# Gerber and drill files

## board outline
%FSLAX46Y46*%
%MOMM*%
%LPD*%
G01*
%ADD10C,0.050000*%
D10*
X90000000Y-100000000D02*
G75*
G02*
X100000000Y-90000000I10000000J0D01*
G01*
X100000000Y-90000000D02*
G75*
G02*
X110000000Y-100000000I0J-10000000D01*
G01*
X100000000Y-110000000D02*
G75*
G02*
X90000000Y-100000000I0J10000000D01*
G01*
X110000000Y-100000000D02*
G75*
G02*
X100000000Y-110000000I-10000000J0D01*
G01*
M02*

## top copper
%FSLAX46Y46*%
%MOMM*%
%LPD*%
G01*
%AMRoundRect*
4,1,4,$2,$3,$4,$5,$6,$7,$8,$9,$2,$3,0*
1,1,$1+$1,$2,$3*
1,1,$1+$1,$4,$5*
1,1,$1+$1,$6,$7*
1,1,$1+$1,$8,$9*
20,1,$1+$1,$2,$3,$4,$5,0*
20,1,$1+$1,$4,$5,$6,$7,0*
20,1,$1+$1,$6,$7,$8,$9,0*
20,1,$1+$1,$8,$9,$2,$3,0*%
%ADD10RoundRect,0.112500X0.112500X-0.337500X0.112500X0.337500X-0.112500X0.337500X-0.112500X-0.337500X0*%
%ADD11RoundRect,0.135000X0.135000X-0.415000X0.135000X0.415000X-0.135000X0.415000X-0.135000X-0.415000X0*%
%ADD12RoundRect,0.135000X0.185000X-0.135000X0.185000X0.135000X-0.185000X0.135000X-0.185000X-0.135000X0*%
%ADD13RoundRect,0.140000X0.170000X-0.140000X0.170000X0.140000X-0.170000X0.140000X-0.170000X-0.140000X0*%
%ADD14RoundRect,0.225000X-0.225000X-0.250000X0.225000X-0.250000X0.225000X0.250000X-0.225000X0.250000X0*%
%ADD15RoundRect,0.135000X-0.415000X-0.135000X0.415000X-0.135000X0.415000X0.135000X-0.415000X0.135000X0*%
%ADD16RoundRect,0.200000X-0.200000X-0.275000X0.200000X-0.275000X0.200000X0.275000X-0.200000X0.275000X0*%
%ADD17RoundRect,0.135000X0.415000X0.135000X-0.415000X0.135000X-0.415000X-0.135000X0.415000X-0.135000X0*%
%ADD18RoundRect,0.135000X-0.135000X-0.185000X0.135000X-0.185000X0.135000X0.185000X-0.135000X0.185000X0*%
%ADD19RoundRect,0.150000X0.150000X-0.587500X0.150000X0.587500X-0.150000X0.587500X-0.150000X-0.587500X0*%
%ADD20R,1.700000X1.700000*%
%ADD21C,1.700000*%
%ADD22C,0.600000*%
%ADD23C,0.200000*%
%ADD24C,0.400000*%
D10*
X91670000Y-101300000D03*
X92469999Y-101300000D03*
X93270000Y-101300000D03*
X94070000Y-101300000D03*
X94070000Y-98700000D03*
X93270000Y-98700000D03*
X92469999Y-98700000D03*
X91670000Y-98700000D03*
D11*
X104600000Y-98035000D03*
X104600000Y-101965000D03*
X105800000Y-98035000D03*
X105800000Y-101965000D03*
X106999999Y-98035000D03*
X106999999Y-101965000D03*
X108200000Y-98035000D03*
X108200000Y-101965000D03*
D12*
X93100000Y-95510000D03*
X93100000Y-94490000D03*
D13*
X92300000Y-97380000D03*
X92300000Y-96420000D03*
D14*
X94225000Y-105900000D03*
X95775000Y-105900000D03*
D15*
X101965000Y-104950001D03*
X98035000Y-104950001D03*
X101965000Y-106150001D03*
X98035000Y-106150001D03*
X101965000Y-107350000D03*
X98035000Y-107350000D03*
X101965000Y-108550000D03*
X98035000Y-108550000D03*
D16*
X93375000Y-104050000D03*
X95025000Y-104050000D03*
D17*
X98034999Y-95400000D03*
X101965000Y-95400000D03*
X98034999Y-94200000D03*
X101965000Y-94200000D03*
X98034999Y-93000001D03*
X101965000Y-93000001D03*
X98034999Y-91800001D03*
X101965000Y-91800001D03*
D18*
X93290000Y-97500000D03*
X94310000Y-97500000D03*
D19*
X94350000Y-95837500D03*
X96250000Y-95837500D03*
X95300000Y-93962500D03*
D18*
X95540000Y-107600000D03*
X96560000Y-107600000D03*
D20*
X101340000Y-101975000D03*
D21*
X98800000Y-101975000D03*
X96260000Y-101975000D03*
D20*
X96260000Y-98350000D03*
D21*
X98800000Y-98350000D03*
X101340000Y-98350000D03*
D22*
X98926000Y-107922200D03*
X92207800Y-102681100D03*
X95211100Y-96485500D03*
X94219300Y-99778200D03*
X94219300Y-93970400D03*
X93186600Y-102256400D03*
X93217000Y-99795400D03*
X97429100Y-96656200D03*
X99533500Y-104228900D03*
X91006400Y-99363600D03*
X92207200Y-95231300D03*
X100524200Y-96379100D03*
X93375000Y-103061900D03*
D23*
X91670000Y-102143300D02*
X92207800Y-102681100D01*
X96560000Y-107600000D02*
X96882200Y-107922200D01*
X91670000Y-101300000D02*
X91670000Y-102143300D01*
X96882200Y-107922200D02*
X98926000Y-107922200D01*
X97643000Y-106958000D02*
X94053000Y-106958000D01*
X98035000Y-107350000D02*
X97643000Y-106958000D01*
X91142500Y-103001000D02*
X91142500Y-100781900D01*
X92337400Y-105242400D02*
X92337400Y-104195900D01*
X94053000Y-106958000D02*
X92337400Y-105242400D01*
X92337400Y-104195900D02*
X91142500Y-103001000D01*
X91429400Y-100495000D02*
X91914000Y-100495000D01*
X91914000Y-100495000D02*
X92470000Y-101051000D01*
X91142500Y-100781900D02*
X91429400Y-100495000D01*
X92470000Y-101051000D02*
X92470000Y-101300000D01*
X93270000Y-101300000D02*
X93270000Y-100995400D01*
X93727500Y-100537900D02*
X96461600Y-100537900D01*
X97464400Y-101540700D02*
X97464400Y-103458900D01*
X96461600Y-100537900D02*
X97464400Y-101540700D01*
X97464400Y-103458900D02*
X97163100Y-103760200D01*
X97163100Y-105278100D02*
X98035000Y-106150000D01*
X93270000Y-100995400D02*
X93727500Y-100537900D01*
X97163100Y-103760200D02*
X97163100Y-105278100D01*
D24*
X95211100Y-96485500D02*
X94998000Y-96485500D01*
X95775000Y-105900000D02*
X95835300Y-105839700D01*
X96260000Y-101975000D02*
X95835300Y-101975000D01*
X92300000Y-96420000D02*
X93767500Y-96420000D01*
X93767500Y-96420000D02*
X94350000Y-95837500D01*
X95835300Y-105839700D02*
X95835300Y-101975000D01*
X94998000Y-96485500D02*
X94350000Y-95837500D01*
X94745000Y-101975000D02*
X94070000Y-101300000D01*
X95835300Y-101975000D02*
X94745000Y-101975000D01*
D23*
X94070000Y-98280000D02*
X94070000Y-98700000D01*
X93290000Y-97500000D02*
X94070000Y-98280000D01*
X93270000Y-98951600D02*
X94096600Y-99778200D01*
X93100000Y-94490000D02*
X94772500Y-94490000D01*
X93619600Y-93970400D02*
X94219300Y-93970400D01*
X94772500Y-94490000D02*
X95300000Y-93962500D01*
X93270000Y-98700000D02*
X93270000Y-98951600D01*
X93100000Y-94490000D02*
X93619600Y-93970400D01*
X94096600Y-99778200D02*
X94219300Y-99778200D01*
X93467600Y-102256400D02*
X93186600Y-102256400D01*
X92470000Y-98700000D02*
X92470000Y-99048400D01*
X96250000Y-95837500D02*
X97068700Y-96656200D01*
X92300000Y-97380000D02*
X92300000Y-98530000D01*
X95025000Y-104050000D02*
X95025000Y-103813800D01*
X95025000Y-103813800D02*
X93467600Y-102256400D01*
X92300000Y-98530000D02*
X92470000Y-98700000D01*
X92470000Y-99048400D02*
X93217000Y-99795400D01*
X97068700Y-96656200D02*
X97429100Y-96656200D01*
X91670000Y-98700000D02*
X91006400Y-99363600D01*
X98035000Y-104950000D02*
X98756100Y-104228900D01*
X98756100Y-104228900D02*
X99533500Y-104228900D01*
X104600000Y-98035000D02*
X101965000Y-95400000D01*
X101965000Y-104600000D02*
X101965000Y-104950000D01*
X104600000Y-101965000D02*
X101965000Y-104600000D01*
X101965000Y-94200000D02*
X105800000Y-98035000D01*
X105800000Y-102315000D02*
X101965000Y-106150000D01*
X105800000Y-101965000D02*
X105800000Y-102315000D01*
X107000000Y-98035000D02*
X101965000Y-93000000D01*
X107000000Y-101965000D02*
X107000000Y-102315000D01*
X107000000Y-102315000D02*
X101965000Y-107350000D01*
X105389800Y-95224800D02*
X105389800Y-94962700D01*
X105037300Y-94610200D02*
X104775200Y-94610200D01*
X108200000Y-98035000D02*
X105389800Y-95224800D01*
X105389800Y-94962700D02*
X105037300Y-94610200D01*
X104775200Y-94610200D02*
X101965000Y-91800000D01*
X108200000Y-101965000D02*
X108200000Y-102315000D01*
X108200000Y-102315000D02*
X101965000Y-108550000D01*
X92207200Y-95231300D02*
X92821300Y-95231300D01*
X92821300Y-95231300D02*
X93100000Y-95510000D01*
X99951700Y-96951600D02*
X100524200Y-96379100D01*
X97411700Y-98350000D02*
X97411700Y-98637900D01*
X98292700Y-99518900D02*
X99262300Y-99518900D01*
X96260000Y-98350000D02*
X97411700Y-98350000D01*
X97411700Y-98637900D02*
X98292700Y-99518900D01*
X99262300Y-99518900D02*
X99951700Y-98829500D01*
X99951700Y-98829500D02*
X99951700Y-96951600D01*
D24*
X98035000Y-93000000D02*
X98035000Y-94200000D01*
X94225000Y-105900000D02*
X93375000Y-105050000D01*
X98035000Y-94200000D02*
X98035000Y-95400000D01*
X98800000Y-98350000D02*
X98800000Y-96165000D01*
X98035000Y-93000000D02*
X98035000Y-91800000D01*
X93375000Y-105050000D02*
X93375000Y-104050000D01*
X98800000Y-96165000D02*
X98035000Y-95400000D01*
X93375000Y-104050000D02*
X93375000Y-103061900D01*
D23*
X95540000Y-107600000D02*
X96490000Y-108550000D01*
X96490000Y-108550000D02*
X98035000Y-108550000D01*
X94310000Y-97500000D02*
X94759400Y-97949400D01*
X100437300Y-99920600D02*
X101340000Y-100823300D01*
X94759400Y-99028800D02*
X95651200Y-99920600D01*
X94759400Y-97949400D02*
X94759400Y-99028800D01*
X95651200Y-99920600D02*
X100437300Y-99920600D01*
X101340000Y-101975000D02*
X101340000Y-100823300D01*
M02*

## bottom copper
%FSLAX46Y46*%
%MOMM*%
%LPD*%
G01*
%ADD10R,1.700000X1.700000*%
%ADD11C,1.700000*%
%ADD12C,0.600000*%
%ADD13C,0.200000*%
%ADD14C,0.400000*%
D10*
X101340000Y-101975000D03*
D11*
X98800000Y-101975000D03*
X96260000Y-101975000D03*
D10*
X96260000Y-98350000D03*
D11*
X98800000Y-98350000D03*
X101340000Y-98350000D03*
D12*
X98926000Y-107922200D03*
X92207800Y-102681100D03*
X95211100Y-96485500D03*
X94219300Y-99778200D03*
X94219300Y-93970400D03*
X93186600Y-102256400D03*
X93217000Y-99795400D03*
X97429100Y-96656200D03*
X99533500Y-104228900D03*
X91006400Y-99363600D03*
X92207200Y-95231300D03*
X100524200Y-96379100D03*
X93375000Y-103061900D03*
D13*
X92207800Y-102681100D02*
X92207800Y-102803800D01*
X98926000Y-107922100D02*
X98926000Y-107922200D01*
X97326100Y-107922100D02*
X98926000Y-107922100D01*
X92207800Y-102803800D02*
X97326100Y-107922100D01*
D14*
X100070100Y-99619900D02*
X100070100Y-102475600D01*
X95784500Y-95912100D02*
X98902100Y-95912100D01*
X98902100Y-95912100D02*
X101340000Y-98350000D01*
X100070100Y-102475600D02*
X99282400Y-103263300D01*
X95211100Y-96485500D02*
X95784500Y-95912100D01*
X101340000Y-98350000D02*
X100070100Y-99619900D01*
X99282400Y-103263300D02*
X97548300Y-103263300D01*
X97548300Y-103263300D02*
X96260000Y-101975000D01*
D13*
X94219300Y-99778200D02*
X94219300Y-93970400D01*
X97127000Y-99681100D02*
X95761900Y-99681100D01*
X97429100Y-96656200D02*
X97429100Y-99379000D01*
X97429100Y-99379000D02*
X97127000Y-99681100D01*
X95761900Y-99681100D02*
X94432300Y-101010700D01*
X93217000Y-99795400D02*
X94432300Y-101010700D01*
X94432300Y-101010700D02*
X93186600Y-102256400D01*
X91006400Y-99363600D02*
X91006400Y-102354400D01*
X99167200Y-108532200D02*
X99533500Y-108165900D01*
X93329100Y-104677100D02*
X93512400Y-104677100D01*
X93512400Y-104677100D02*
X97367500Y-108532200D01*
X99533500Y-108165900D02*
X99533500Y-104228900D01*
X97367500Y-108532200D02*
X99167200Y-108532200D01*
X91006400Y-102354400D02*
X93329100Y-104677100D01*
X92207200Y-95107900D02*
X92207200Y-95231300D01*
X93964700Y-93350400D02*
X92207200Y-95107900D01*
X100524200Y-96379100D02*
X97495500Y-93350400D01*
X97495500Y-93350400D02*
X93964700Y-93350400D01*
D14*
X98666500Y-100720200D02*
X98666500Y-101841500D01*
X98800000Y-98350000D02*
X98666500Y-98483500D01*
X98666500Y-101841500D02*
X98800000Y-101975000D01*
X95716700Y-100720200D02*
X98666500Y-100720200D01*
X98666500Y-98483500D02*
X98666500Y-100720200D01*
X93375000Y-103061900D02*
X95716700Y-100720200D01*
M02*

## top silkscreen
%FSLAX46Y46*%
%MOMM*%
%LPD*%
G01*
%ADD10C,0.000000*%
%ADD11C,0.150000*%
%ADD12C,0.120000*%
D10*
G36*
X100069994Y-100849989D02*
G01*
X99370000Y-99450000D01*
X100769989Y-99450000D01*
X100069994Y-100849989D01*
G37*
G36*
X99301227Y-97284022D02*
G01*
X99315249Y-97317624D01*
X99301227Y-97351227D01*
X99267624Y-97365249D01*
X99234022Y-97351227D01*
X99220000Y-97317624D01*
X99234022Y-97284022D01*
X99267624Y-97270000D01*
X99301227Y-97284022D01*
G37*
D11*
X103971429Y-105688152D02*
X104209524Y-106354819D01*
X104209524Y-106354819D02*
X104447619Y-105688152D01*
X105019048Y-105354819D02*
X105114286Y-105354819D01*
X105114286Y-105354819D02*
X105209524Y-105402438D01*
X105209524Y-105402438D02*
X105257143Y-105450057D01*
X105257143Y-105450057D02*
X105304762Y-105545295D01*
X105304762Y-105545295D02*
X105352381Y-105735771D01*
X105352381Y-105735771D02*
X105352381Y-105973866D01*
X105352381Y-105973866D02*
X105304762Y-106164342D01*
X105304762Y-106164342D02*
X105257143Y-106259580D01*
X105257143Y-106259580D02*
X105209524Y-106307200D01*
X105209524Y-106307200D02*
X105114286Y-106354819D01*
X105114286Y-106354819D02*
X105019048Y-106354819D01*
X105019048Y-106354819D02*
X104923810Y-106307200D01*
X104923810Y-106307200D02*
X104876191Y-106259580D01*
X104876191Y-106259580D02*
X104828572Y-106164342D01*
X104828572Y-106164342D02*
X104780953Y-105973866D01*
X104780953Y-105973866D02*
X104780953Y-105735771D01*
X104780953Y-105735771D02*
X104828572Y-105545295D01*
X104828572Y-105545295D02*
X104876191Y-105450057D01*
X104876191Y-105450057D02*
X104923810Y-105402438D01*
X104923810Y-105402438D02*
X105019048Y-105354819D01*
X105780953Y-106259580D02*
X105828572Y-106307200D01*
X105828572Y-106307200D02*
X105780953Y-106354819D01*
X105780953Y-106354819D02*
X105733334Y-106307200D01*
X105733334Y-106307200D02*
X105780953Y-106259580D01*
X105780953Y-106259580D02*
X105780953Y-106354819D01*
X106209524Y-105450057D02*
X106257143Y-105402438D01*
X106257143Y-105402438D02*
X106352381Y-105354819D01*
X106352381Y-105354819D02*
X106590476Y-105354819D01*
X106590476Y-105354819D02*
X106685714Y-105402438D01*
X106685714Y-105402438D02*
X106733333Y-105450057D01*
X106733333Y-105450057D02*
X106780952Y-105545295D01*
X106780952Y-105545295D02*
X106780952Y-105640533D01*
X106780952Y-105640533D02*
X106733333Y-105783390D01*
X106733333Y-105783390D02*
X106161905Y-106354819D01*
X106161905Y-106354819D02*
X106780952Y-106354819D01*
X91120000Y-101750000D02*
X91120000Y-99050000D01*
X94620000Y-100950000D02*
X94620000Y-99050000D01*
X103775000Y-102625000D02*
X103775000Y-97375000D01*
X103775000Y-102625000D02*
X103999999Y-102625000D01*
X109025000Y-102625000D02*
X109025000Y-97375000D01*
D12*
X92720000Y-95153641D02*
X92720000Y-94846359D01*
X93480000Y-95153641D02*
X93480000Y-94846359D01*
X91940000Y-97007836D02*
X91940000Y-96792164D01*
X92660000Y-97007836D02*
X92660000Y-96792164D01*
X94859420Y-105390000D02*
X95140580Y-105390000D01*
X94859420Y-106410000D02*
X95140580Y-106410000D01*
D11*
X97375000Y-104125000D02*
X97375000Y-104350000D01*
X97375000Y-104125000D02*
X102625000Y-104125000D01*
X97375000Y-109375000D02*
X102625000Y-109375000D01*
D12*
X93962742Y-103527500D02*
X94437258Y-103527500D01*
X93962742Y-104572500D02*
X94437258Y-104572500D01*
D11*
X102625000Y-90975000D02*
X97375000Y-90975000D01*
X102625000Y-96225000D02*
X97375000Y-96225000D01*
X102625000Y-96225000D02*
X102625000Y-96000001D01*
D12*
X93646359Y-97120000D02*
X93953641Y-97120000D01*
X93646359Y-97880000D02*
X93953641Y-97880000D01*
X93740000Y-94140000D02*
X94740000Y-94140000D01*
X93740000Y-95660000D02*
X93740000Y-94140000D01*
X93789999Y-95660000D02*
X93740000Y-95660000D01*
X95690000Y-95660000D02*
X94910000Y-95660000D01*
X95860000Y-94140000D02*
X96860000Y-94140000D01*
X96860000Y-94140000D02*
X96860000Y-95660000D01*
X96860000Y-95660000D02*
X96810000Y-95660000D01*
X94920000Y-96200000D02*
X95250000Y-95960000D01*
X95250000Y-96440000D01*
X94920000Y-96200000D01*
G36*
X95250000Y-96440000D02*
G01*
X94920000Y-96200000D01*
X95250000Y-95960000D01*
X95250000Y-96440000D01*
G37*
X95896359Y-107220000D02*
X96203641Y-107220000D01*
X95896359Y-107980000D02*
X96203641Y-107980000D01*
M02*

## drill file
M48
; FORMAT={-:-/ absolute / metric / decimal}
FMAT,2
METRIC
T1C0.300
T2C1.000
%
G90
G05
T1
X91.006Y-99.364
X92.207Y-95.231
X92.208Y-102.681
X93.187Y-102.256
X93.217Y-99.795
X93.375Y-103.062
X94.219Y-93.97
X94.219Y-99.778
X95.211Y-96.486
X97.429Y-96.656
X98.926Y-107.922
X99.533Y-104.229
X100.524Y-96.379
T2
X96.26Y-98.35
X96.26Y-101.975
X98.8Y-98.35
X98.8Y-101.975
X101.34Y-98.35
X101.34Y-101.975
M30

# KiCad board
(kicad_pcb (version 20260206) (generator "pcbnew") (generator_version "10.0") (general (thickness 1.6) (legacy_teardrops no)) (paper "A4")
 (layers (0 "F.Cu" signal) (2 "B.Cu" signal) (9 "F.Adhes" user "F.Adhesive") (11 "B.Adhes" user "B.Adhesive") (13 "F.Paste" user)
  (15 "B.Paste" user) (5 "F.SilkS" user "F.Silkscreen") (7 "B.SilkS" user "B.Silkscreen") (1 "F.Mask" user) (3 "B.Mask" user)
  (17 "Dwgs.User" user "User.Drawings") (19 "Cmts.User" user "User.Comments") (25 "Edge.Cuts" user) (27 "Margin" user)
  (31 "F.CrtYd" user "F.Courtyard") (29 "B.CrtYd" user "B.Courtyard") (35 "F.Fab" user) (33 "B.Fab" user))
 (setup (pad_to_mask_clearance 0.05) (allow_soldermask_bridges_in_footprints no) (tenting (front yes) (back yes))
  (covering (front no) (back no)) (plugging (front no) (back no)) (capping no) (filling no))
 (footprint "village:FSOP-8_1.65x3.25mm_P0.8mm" (layer "F.Cu") (at 92.87 100 90)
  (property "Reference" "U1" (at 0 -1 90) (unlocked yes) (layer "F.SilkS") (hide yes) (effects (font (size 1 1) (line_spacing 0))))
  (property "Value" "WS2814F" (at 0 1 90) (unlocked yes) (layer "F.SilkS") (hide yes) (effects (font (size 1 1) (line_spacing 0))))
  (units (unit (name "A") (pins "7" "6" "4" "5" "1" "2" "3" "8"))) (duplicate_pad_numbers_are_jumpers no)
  (fp_line (start -1.75 -1.75) (end 0.95 -1.75) (stroke (width 0.15) (type solid)) (layer "F.SilkS"))
  (fp_line (start -0.95 1.75) (end 0.95 1.75) (stroke (width 0.15) (type solid)) (layer "F.SilkS"))
  (pad "1" smd roundrect (at -1.3 -1.2 90) (size 0.9 0.45) (layers "F.Cu" "F.Mask" "F.Paste") (roundrect_rratio 0.25) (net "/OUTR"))
  (pad "2" smd roundrect (at -1.3 -0.400001 90) (size 0.9 0.45) (layers "F.Cu" "F.Mask" "F.Paste") (roundrect_rratio 0.25) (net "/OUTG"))
  (pad "3" smd roundrect (at -1.3 0.4 90) (size 0.9 0.45) (layers "F.Cu" "F.Mask" "F.Paste") (roundrect_rratio 0.25) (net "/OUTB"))
  (pad "4" smd roundrect (at -1.3 1.2 90) (size 0.9 0.45) (layers "F.Cu" "F.Mask" "F.Paste") (roundrect_rratio 0.25) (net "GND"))
  (pad "5" smd roundrect (at 1.3 1.2 90) (size 0.9 0.45) (layers "F.Cu" "F.Mask" "F.Paste") (roundrect_rratio 0.25) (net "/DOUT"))
  (pad "6" smd roundrect (at 1.3 0.4 90) (size 0.9 0.45) (layers "F.Cu" "F.Mask" "F.Paste") (roundrect_rratio 0.25) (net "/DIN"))
  (pad "7" smd roundrect (at 1.3 -0.400001 90) (size 0.9 0.45) (layers "F.Cu" "F.Mask" "F.Paste") (roundrect_rratio 0.25) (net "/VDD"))
  (pad "8" smd roundrect (at 1.3 -1.2 90) (size 0.9 0.45) (layers "F.Cu" "F.Mask" "F.Paste") (roundrect_rratio 0.25) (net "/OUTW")))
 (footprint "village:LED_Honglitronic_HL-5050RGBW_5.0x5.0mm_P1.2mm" (layer "F.Cu") (at 106.4 100 90)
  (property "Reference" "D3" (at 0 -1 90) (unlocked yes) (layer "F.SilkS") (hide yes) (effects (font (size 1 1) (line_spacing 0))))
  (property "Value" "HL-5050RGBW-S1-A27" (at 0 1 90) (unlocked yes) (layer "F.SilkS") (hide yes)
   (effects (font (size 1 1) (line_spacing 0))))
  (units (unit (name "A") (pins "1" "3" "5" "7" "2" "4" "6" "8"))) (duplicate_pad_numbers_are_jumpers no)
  (fp_line (start -2.625 -2.625) (end 2.625 -2.625) (stroke (width 0.15) (type default)) (layer "F.SilkS"))
  (fp_line (start -2.625 -2.625) (end -2.625 -2.400001) (stroke (width 0.15) (type default)) (layer "F.SilkS"))
  (fp_line (start -2.625 2.625) (end 2.625 2.625) (stroke (width 0.15) (type default)) (layer "F.SilkS"))
  (pad "1" smd roundrect (at 1.965 -1.8 90) (size 1.1 0.54) (layers "F.Cu" "F.Mask" "F.Paste") (roundrect_rratio 0.25) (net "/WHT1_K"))
  (pad "2" smd roundrect (at -1.965 -1.8 90) (size 1.1 0.54) (layers "F.Cu" "F.Mask" "F.Paste") (roundrect_rratio 0.25) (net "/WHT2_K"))
  (pad "3" smd roundrect (at 1.965 -0.6 90) (size 1.1 0.54) (layers "F.Cu" "F.Mask" "F.Paste") (roundrect_rratio 0.25) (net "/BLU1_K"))
  (pad "4" smd roundrect (at -1.965 -0.6 90) (size 1.1 0.54) (layers "F.Cu" "F.Mask" "F.Paste") (roundrect_rratio 0.25) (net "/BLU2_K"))
  (pad "5" smd roundrect (at 1.965 0.599999 90) (size 1.1 0.54) (layers "F.Cu" "F.Mask" "F.Paste") (roundrect_rratio 0.25) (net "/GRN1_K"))
  (pad "6" smd roundrect (at -1.965 0.599999 90) (size 1.1 0.54) (layers "F.Cu" "F.Mask" "F.Paste") (roundrect_rratio 0.25) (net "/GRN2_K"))
  (pad "7" smd roundrect (at 1.965 1.8 90) (size 1.1 0.54) (layers "F.Cu" "F.Mask" "F.Paste") (roundrect_rratio 0.25) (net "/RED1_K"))
  (pad "8" smd roundrect (at -1.965 1.8 90) (size 1.1 0.54) (layers "F.Cu" "F.Mask" "F.Paste") (roundrect_rratio 0.25) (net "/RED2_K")))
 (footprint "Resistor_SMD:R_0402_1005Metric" (layer "F.Cu") (at 93.1 95 90)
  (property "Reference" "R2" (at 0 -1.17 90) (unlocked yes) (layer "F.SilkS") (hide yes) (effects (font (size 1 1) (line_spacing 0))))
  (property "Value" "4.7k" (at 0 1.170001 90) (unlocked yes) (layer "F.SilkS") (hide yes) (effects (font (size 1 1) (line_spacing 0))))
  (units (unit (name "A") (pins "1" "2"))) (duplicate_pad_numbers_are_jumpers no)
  (fp_line (start -0.153641 -0.38) (end 0.153641 -0.38) (stroke (width 0.12) (type solid)) (layer "F.SilkS"))
  (fp_line (start -0.153641 0.38) (end 0.153641 0.38) (stroke (width 0.12) (type solid)) (layer "F.SilkS"))
  (pad "1" smd roundrect (at -0.51 0 90) (size 0.54 0.64) (layers "F.Cu" "F.Mask" "F.Paste") (roundrect_rratio 0.25) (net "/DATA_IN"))
  (pad "2" smd roundrect (at 0.51 0 90) (size 0.54 0.64) (layers "F.Cu" "F.Mask" "F.Paste") (roundrect_rratio 0.25) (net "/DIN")))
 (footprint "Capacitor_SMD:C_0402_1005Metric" (layer "F.Cu") (at 92.3 96.9 90)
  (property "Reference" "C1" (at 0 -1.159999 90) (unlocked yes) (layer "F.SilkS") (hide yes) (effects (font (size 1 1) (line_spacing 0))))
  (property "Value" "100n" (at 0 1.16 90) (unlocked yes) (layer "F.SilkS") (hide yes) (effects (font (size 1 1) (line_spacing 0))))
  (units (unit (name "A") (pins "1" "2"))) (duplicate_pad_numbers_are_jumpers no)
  (fp_line (start -0.107836 -0.36) (end 0.107836 -0.36) (stroke (width 0.12) (type solid)) (layer "F.SilkS"))
  (fp_line (start -0.107836 0.36) (end 0.107836 0.36) (stroke (width 0.12) (type solid)) (layer "F.SilkS"))
  (pad "1" smd roundrect (at -0.48 0 90) (size 0.56 0.62) (layers "F.Cu" "F.Mask" "F.Paste") (roundrect_rratio 0.25) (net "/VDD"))
  (pad "2" smd roundrect (at 0.48 0 90) (size 0.56 0.62) (layers "F.Cu" "F.Mask" "F.Paste") (roundrect_rratio 0.25) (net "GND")))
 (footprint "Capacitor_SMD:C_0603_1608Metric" (layer "F.Cu") (at 95 105.9)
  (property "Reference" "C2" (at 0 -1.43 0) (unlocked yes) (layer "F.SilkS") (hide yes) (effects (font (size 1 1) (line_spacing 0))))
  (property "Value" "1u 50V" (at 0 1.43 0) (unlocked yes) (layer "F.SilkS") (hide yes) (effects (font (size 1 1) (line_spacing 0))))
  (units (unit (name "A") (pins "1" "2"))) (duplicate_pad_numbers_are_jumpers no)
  (fp_line (start -0.14058 -0.51) (end 0.14058 -0.51) (stroke (width 0.12) (type solid)) (layer "F.SilkS"))
  (fp_line (start -0.14058 0.51) (end 0.14058 0.51) (stroke (width 0.12) (type solid)) (layer "F.SilkS"))
  (pad "1" smd roundrect (at -0.775 0) (size 0.9 0.95) (layers "F.Cu" "F.Mask" "F.Paste") (roundrect_rratio 0.25) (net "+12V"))
  (pad "2" smd roundrect (at 0.775 0) (size 0.9 0.95) (layers "F.Cu" "F.Mask" "F.Paste") (roundrect_rratio 0.25) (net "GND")))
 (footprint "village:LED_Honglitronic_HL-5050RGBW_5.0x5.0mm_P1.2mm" (layer "F.Cu") (at 100 106.75)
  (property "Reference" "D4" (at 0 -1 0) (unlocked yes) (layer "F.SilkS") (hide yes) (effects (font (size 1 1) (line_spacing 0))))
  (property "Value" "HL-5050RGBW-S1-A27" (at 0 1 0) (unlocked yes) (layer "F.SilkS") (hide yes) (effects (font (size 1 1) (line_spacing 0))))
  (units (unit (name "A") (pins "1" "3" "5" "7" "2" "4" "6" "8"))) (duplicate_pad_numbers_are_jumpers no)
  (fp_line (start -2.625 -2.625) (end -2.625 -2.4) (stroke (width 0.15) (type default)) (layer "F.SilkS"))
  (fp_line (start -2.625 -2.625) (end 2.625 -2.625) (stroke (width 0.15) (type default)) (layer "F.SilkS"))
  (fp_line (start -2.625 2.625) (end 2.625 2.625) (stroke (width 0.15) (type default)) (layer "F.SilkS"))
  (pad "1" smd roundrect (at 1.965 -1.799999) (size 1.1 0.54) (layers "F.Cu" "F.Mask" "F.Paste") (roundrect_rratio 0.25) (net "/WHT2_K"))
  (pad "2" smd roundrect (at -1.965 -1.799999) (size 1.1 0.54) (layers "F.Cu" "F.Mask" "F.Paste") (roundrect_rratio 0.25) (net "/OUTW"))
  (pad "3" smd roundrect (at 1.965 -0.599999) (size 1.1 0.54) (layers "F.Cu" "F.Mask" "F.Paste") (roundrect_rratio 0.25) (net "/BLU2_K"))
  (pad "4" smd roundrect (at -1.965 -0.599999) (size 1.1 0.54) (layers "F.Cu" "F.Mask" "F.Paste") (roundrect_rratio 0.25) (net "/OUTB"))
  (pad "5" smd roundrect (at 1.965 0.6) (size 1.1 0.54) (layers "F.Cu" "F.Mask" "F.Paste") (roundrect_rratio 0.25) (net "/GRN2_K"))
  (pad "6" smd roundrect (at -1.965 0.6) (size 1.1 0.54) (layers "F.Cu" "F.Mask" "F.Paste") (roundrect_rratio 0.25) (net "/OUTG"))
  (pad "7" smd roundrect (at 1.965 1.8) (size 1.1 0.54) (layers "F.Cu" "F.Mask" "F.Paste") (roundrect_rratio 0.25) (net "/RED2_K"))
  (pad "8" smd roundrect (at -1.965 1.8) (size 1.1 0.54) (layers "F.Cu" "F.Mask" "F.Paste") (roundrect_rratio 0.25) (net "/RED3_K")))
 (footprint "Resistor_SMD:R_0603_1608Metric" (layer "F.Cu") (at 94.2 104.05)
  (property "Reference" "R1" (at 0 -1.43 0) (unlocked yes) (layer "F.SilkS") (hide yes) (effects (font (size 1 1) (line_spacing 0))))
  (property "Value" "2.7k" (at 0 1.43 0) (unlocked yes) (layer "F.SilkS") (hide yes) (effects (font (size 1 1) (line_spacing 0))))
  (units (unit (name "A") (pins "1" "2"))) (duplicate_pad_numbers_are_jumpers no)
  (fp_line (start -0.237258 -0.5225) (end 0.237258 -0.5225) (stroke (width 0.12) (type solid)) (layer "F.SilkS"))
  (fp_line (start -0.237258 0.5225) (end 0.237258 0.5225) (stroke (width 0.12) (type solid)) (layer "F.SilkS"))
  (pad "1" smd roundrect (at -0.825 0) (size 0.8 0.95) (layers "F.Cu" "F.Mask" "F.Paste") (roundrect_rratio 0.25) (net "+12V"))
  (pad "2" smd roundrect (at 0.825 0) (size 0.8 0.95) (layers "F.Cu" "F.Mask" "F.Paste") (roundrect_rratio 0.25) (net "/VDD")))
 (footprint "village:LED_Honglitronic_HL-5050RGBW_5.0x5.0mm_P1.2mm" (layer "F.Cu") (at 100 93.6 180)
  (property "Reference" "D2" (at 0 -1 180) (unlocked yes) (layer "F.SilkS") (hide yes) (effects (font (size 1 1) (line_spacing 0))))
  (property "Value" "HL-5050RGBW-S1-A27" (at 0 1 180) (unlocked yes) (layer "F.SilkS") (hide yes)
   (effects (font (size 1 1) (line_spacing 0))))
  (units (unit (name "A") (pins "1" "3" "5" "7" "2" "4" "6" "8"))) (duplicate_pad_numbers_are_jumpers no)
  (fp_line (start -2.625 2.625) (end 2.625 2.625) (stroke (width 0.15) (type default)) (layer "F.SilkS"))
  (fp_line (start -2.625 -2.625) (end 2.625 -2.625) (stroke (width 0.15) (type default)) (layer "F.SilkS"))
  (fp_line (start -2.625 -2.625) (end -2.625 -2.400001) (stroke (width 0.15) (type default)) (layer "F.SilkS"))
  (pad "1" smd roundrect (at 1.965001 -1.8 180) (size 1.1 0.54) (layers "F.Cu" "F.Mask" "F.Paste") (roundrect_rratio 0.25) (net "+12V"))
  (pad "2" smd roundrect (at -1.965 -1.8 180) (size 1.1 0.54) (layers "F.Cu" "F.Mask" "F.Paste") (roundrect_rratio 0.25) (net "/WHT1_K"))
  (pad "3" smd roundrect (at 1.965001 -0.6 180) (size 1.1 0.54) (layers "F.Cu" "F.Mask" "F.Paste") (roundrect_rratio 0.25) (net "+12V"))
  (pad "4" smd roundrect (at -1.965 -0.6 180) (size 1.1 0.54) (layers "F.Cu" "F.Mask" "F.Paste") (roundrect_rratio 0.25) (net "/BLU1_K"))
  (pad "5" smd roundrect (at 1.965001 0.599999 180) (size 1.1 0.54) (layers "F.Cu" "F.Mask" "F.Paste") (roundrect_rratio 0.25) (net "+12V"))
  (pad "6" smd roundrect (at -1.965 0.599999 180) (size 1.1 0.54) (layers "F.Cu" "F.Mask" "F.Paste") (roundrect_rratio 0.25) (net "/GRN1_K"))
  (pad "7" smd roundrect (at 1.965001 1.799999 180) (size 1.1 0.54) (layers "F.Cu" "F.Mask" "F.Paste") (roundrect_rratio 0.25) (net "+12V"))
  (pad "8" smd roundrect (at -1.965 1.799999 180) (size 1.1 0.54) (layers "F.Cu" "F.Mask" "F.Paste") (roundrect_rratio 0.25) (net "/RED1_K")))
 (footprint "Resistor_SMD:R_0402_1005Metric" (layer "F.Cu") (at 93.8 97.5)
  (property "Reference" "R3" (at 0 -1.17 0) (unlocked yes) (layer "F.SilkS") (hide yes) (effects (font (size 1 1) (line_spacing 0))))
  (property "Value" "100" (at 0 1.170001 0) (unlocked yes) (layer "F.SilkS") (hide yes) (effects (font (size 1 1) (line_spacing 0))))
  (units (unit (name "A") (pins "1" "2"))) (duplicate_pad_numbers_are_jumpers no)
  (fp_line (start -0.153641 -0.38) (end 0.153641 -0.38) (stroke (width 0.12) (type solid)) (layer "F.SilkS"))
  (fp_line (start -0.153641 0.38) (end 0.153641 0.38) (stroke (width 0.12) (type solid)) (layer "F.SilkS"))
  (pad "1" smd roundrect (at -0.51 0) (size 0.54 0.64) (layers "F.Cu" "F.Mask" "F.Paste") (roundrect_rratio 0.25) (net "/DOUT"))
  (pad "2" smd roundrect (at 0.51 0) (size 0.54 0.64) (layers "F.Cu" "F.Mask" "F.Paste") (roundrect_rratio 0.25) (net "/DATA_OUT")))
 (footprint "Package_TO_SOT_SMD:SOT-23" (layer "F.Cu") (at 95.3 94.9 90)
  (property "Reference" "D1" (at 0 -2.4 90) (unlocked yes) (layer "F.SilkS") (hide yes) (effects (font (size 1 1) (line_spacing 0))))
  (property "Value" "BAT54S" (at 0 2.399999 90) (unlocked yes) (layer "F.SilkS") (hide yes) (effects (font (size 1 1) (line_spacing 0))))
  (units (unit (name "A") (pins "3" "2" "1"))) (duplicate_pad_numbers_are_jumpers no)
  (fp_line (start 0.76 -1.56) (end 0.76 -0.56) (stroke (width 0.12) (type solid)) (layer "F.SilkS"))
  (fp_line (start -0.76 -1.56) (end 0.76 -1.56) (stroke (width 0.12) (type solid)) (layer "F.SilkS"))
  (fp_line (start -0.76 -1.510001) (end -0.76 -1.56) (stroke (width 0.12) (type solid)) (layer "F.SilkS"))
  (fp_line (start -0.76 0.39) (end -0.76 -0.39) (stroke (width 0.12) (type solid)) (layer "F.SilkS"))
  (fp_line (start 0.76 0.56) (end 0.76 1.56) (stroke (width 0.12) (type solid)) (layer "F.SilkS"))
  (fp_line (start 0.76 1.56) (end -0.76 1.56) (stroke (width 0.12) (type solid)) (layer "F.SilkS"))
  (fp_line (start -0.76 1.56) (end -0.76 1.51) (stroke (width 0.12) (type solid)) (layer "F.SilkS"))
  (fp_poly (pts (xy -1.3 -0.38) (xy -1.06 -0.05) (xy -1.54 -0.05)) (stroke (width 0.12) (type solid)) (fill yes) (layer "F.SilkS"))
  (pad "1" smd roundrect (at -0.9375 -0.95 90) (size 1.475 0.6) (layers "F.Cu" "F.Mask" "F.Paste") (roundrect_rratio 0.25) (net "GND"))
  (pad "2" smd roundrect (at -0.9375 0.95 90) (size 1.475 0.6) (layers "F.Cu" "F.Mask" "F.Paste") (roundrect_rratio 0.25) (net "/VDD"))
  (pad "3" smd roundrect (at 0.9375 0 90) (size 1.475 0.6) (layers "F.Cu" "F.Mask" "F.Paste") (roundrect_rratio 0.25) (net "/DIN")))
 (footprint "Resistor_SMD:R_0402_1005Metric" (layer "F.Cu") (at 96.05 107.6)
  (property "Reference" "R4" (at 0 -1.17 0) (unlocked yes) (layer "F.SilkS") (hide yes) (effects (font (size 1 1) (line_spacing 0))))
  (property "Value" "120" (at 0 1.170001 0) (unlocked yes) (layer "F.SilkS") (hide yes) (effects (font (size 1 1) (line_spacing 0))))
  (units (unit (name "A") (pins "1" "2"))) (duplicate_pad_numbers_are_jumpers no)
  (fp_line (start -0.153641 -0.38) (end 0.153641 -0.38) (stroke (width 0.12) (type solid)) (layer "F.SilkS"))
  (fp_line (start -0.153641 0.38) (end 0.153641 0.38) (stroke (width 0.12) (type solid)) (layer "F.SilkS"))
  (pad "1" smd roundrect (at -0.51 0) (size 0.54 0.64) (layers "F.Cu" "F.Mask" "F.Paste") (roundrect_rratio 0.25) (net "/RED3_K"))
  (pad "2" smd roundrect (at 0.51 0) (size 0.54 0.64) (layers "F.Cu" "F.Mask" "F.Paste") (roundrect_rratio 0.25) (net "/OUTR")))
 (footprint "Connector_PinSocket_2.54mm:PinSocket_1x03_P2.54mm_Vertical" (layer "B.Cu") (at 101.34 101.975 90)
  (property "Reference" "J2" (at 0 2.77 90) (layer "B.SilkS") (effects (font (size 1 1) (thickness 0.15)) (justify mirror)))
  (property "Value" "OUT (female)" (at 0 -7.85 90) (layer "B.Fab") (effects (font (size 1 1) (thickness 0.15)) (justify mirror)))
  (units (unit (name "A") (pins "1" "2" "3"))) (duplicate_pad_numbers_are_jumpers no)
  (pad "1" thru_hole rect (at 0 0 90) (size 1.7 1.7) (drill 1) (layers "*.Cu" "*.Mask") (remove_unused_layers no) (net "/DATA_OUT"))
  (pad "2" thru_hole circle (at 0 -2.54 90) (size 1.7 1.7) (drill 1) (layers "*.Cu" "*.Mask") (remove_unused_layers no) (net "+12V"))
  (pad "3" thru_hole circle (at 0 -5.08 90) (size 1.7 1.7) (drill 1) (layers "*.Cu" "*.Mask") (remove_unused_layers no) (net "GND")))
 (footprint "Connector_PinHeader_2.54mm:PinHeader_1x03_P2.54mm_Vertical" (layer "B.Cu") (at 96.26 98.35 -90)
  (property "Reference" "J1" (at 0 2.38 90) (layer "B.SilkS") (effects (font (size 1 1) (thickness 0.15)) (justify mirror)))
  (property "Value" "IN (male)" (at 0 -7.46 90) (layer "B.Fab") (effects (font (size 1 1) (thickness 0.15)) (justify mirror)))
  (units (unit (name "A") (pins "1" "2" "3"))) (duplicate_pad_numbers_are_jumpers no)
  (pad "1" thru_hole rect (at 0 0 270) (size 1.7 1.7) (drill 1) (layers "*.Cu" "*.Mask") (remove_unused_layers no) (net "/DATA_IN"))
  (pad "2" thru_hole circle (at 0 -2.54 270) (size 1.7 1.7) (drill 1) (layers "*.Cu" "*.Mask") (remove_unused_layers no) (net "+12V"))
  (pad "3" thru_hole circle (at 0 -5.08 270) (size 1.7 1.7) (drill 1) (layers "*.Cu" "*.Mask") (remove_unused_layers no) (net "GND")))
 (gr_poly
  (pts (xy 99.37 99.45) (xy 100.769989 99.45) (xy 100.069994 100.849989)) (stroke (width 0) (type default)) (fill yes) (layer "F.SilkS"))
 (gr_poly
  (pts (xy 99.267624 97.27) (xy 99.301227 97.284022) (xy 99.315249 97.317624) (xy 99.301227 97.351227) (xy 99.267624 97.365249)
   (xy 99.234022 97.351227) (xy 99.22 97.317624) (xy 99.234022 97.284022))
  (stroke (width 0) (type default)) (fill yes) (layer "F.SilkS"))
 (gr_arc (start 90 100) (mid 92.928932 92.928932) (end 100 90) (stroke (width 0.05) (type solid)) (layer "Edge.Cuts"))
 (gr_arc (start 100 90) (mid 107.071068 92.928932) (end 110 100) (stroke (width 0.05) (type solid)) (layer "Edge.Cuts"))
 (gr_arc (start 100 110) (mid 92.928932 107.071068) (end 90 100) (stroke (width 0.05) (type solid)) (layer "Edge.Cuts"))
 (gr_arc (start 110 100) (mid 107.071068 107.071068) (end 100 110) (stroke (width 0.05) (type solid)) (layer "Edge.Cuts"))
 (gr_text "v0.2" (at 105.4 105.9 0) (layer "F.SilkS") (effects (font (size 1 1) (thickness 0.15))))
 (segment (start 91.67 102.1433) (end 92.2078 102.6811) (width 0.2) (layer "F.Cu") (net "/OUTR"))
 (segment (start 96.56 107.6) (end 96.8822 107.9222) (width 0.2) (layer "F.Cu") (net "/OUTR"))
 (segment (start 91.67 101.3) (end 91.67 102.1433) (width 0.2) (layer "F.Cu") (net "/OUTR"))
 (segment (start 96.8822 107.9222) (end 98.926 107.9222) (width 0.2) (layer "F.Cu") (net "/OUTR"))
 (via (at 98.926 107.9222) (size 0.6) (drill 0.3) (layers "F.Cu" "B.Cu") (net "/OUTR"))
 (via (at 92.2078 102.6811) (size 0.6) (drill 0.3) (layers "F.Cu" "B.Cu") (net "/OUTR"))
 (segment (start 92.2078 102.6811) (end 92.2078 102.8038) (width 0.2) (layer "B.Cu") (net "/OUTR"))
 (segment (start 98.926 107.9221) (end 98.926 107.9222) (width 0.2) (layer "B.Cu") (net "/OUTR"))
 (segment (start 97.3261 107.9221) (end 98.926 107.9221) (width 0.2) (layer "B.Cu") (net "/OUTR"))
 (segment (start 92.2078 102.8038) (end 97.3261 107.9221) (width 0.2) (layer "B.Cu") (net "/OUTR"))
 (segment (start 97.643 106.958) (end 94.053 106.958) (width 0.2) (layer "F.Cu") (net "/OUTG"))
 (segment (start 98.035 107.35) (end 97.643 106.958) (width 0.2) (layer "F.Cu") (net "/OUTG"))
 (segment (start 91.1425 103.001) (end 91.1425 100.7819) (width 0.2) (layer "F.Cu") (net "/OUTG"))
 (segment (start 92.3374 105.2424) (end 92.3374 104.1959) (width 0.2) (layer "F.Cu") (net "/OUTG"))
 (segment (start 94.053 106.958) (end 92.3374 105.2424) (width 0.2) (layer "F.Cu") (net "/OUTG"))
 (segment (start 92.3374 104.1959) (end 91.1425 103.001) (width 0.2) (layer "F.Cu") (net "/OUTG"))
 (segment (start 91.4294 100.495) (end 91.914 100.495) (width 0.2) (layer "F.Cu") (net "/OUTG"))
 (segment (start 91.914 100.495) (end 92.47 101.051) (width 0.2) (layer "F.Cu") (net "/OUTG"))
 (segment (start 91.1425 100.7819) (end 91.4294 100.495) (width 0.2) (layer "F.Cu") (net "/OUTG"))
 (segment (start 92.47 101.051) (end 92.47 101.3) (width 0.2) (layer "F.Cu") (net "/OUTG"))
 (segment (start 93.27 101.3) (end 93.27 100.9954) (width 0.2) (layer "F.Cu") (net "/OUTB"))
 (segment (start 93.7275 100.5379) (end 96.4616 100.5379) (width 0.2) (layer "F.Cu") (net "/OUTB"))
 (segment (start 97.4644 101.5407) (end 97.4644 103.4589) (width 0.2) (layer "F.Cu") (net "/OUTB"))
 (segment (start 96.4616 100.5379) (end 97.4644 101.5407) (width 0.2) (layer "F.Cu") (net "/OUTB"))
 (segment (start 97.4644 103.4589) (end 97.1631 103.7602) (width 0.2) (layer "F.Cu") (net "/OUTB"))
 (segment (start 97.1631 105.2781) (end 98.035 106.15) (width 0.2) (layer "F.Cu") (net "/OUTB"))
 (segment (start 93.27 100.9954) (end 93.7275 100.5379) (width 0.2) (layer "F.Cu") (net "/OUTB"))
 (segment (start 97.1631 103.7602) (end 97.1631 105.2781) (width 0.2) (layer "F.Cu") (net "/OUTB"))
 (segment (start 95.2111 96.4855) (end 94.998 96.4855) (width 0.4) (layer "F.Cu") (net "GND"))
 (segment (start 95.775 105.9) (end 95.8353 105.8397) (width 0.4) (layer "F.Cu") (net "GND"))
 (segment (start 96.26 101.975) (end 95.8353 101.975) (width 0.4) (layer "F.Cu") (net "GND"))
 (segment (start 92.3 96.42) (end 93.7675 96.42) (width 0.4) (layer "F.Cu") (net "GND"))
 (segment (start 93.7675 96.42) (end 94.35 95.8375) (width 0.4) (layer "F.Cu") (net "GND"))
 (segment (start 95.8353 105.8397) (end 95.8353 101.975) (width 0.4) (layer "F.Cu") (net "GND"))
 (segment (start 94.998 96.4855) (end 94.35 95.8375) (width 0.4) (layer "F.Cu") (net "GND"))
 (segment (start 94.745 101.975) (end 94.07 101.3) (width 0.4) (layer "F.Cu") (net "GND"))
 (segment (start 95.8353 101.975) (end 94.745 101.975) (width 0.4) (layer "F.Cu") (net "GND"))
 (via (at 95.2111 96.4855) (size 0.6) (drill 0.3) (layers "F.Cu" "B.Cu") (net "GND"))
 (segment (start 100.0701 99.6199) (end 100.0701 102.4756) (width 0.4) (layer "B.Cu") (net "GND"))
 (segment (start 95.7845 95.9121) (end 98.9021 95.9121) (width 0.4) (layer "B.Cu") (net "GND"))
 (segment (start 98.9021 95.9121) (end 101.34 98.35) (width 0.4) (layer "B.Cu") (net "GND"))
 (segment (start 100.0701 102.4756) (end 99.2824 103.2633) (width 0.4) (layer "B.Cu") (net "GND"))
 (segment (start 95.2111 96.4855) (end 95.7845 95.9121) (width 0.4) (layer "B.Cu") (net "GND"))
 (segment (start 101.34 98.35) (end 100.0701 99.6199) (width 0.4) (layer "B.Cu") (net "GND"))
 (segment (start 99.2824 103.2633) (end 97.5483 103.2633) (width 0.4) (layer "B.Cu") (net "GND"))
 (segment (start 97.5483 103.2633) (end 96.26 101.975) (width 0.4) (layer "B.Cu") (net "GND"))
 (segment (start 94.07 98.28) (end 94.07 98.7) (width 0.2) (layer "F.Cu") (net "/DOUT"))
 (segment (start 93.29 97.5) (end 94.07 98.28) (width 0.2) (layer "F.Cu") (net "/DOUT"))
 (segment (start 93.27 98.9516) (end 94.0966 99.7782) (width 0.2) (layer "F.Cu") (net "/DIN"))
 (segment (start 93.1 94.49) (end 94.7725 94.49) (width 0.2) (layer "F.Cu") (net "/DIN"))
 (segment (start 93.6196 93.9704) (end 94.2193 93.9704) (width 0.2) (layer "F.Cu") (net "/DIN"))
 (segment (start 94.7725 94.49) (end 95.3 93.9625) (width 0.2) (layer "F.Cu") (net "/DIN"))
 (segment (start 93.27 98.7) (end 93.27 98.9516) (width 0.2) (layer "F.Cu") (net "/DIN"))
 (segment (start 93.1 94.49) (end 93.6196 93.9704) (width 0.2) (layer "F.Cu") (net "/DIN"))
 (segment (start 94.0966 99.7782) (end 94.2193 99.7782) (width 0.2) (layer "F.Cu") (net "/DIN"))
 (via (at 94.2193 99.7782) (size 0.6) (drill 0.3) (layers "F.Cu" "B.Cu") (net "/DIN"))
 (via (at 94.2193 93.9704) (size 0.6) (drill 0.3) (layers "F.Cu" "B.Cu") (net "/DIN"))
 (segment (start 94.2193 99.7782) (end 94.2193 93.9704) (width 0.2) (layer "B.Cu") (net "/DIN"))
 (segment (start 93.4676 102.2564) (end 93.1866 102.2564) (width 0.2) (layer "F.Cu") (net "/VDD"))
 (segment (start 92.47 98.7) (end 92.47 99.0484) (width 0.2) (layer "F.Cu") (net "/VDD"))
 (segment (start 96.25 95.8375) (end 97.0687 96.6562) (width 0.2) (layer "F.Cu") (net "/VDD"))
 (segment (start 92.3 97.38) (end 92.3 98.53) (width 0.2) (layer "F.Cu") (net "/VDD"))
 (segment (start 95.025 104.05) (end 95.025 103.8138) (width 0.2) (layer "F.Cu") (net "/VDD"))
 (segment (start 95.025 103.8138) (end 93.4676 102.2564) (width 0.2) (layer "F.Cu") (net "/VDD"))
 (segment (start 92.3 98.53) (end 92.47 98.7) (width 0.2) (layer "F.Cu") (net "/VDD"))
 (segment (start 92.47 99.0484) (end 93.217 99.7954) (width 0.2) (layer "F.Cu") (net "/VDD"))
 (segment (start 97.0687 96.6562) (end 97.4291 96.6562) (width 0.2) (layer "F.Cu") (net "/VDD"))
 (via (at 93.1866 102.2564) (size 0.6) (drill 0.3) (layers "F.Cu" "B.Cu") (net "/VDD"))
 (via (at 93.217 99.7954) (size 0.6) (drill 0.3) (layers "F.Cu" "B.Cu") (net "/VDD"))
 (via (at 97.4291 96.6562) (size 0.6) (drill 0.3) (layers "F.Cu" "B.Cu") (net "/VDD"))
 (segment (start 97.127 99.6811) (end 95.7619 99.6811) (width 0.2) (layer "B.Cu") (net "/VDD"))
 (segment (start 97.4291 96.6562) (end 97.4291 99.379) (width 0.2) (layer "B.Cu") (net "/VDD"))
 (segment (start 97.4291 99.379) (end 97.127 99.6811) (width 0.2) (layer "B.Cu") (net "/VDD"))
 (segment (start 95.7619 99.6811) (end 94.4323 101.0107) (width 0.2) (layer "B.Cu") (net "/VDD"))
 (segment (start 93.217 99.7954) (end 94.4323 101.0107) (width 0.2) (layer "B.Cu") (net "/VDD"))
 (segment (start 94.4323 101.0107) (end 93.1866 102.2564) (width 0.2) (layer "B.Cu") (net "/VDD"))
 (segment (start 91.67 98.7) (end 91.0064 99.3636) (width 0.2) (layer "F.Cu") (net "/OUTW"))
 (segment (start 98.035 104.95) (end 98.7561 104.2289) (width 0.2) (layer "F.Cu") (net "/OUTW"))
 (segment (start 98.7561 104.2289) (end 99.5335 104.2289) (width 0.2) (layer "F.Cu") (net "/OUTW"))
 (via (at 99.5335 104.2289) (size 0.6) (drill 0.3) (layers "F.Cu" "B.Cu") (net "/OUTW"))
 (via (at 91.0064 99.3636) (size 0.6) (drill 0.3) (layers "F.Cu" "B.Cu") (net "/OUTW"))
 (segment (start 91.0064 99.3636) (end 91.0064 102.3544) (width 0.2) (layer "B.Cu") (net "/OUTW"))
 (segment (start 99.1672 108.5322) (end 99.5335 108.1659) (width 0.2) (layer "B.Cu") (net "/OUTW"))
 (segment (start 93.3291 104.6771) (end 93.5124 104.6771) (width 0.2) (layer "B.Cu") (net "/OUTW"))
 (segment (start 93.5124 104.6771) (end 97.3675 108.5322) (width 0.2) (layer "B.Cu") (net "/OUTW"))
 (segment (start 99.5335 108.1659) (end 99.5335 104.2289) (width 0.2) (layer "B.Cu") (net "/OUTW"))
 (segment (start 97.3675 108.5322) (end 99.1672 108.5322) (width 0.2) (layer "B.Cu") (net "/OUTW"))
 (segment (start 91.0064 102.3544) (end 93.3291 104.6771) (width 0.2) (layer "B.Cu") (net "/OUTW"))
 (segment (start 104.6 98.035) (end 101.965 95.4) (width 0.2) (layer "F.Cu") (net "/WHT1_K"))
 (segment (start 101.965 104.6) (end 101.965 104.95) (width 0.2) (layer "F.Cu") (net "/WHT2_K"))
 (segment (start 104.6 101.965) (end 101.965 104.6) (width 0.2) (layer "F.Cu") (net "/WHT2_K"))
 (segment (start 101.965 94.2) (end 105.8 98.035) (width 0.2) (layer "F.Cu") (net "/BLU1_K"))
 (segment (start 105.8 102.315) (end 101.965 106.15) (width 0.2) (layer "F.Cu") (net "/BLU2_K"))
 (segment (start 105.8 101.965) (end 105.8 102.315) (width 0.2) (layer "F.Cu") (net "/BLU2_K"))
 (segment (start 107 98.035) (end 101.965 93) (width 0.2) (layer "F.Cu") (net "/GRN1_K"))
 (segment (start 107 101.965) (end 107 102.315) (width 0.2) (layer "F.Cu") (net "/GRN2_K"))
 (segment (start 107 102.315) (end 101.965 107.35) (width 0.2) (layer "F.Cu") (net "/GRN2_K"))
 (segment (start 105.3898 95.2248) (end 105.3898 94.9627) (width 0.2) (layer "F.Cu") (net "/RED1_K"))
 (segment (start 105.0373 94.6102) (end 104.7752 94.6102) (width 0.2) (layer "F.Cu") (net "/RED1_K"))
 (segment (start 108.2 98.035) (end 105.3898 95.2248) (width 0.2) (layer "F.Cu") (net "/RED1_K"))
 (segment (start 105.3898 94.9627) (end 105.0373 94.6102) (width 0.2) (layer "F.Cu") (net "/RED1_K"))
 (segment (start 104.7752 94.6102) (end 101.965 91.8) (width 0.2) (layer "F.Cu") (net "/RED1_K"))
 (segment (start 108.2 101.965) (end 108.2 102.315) (width 0.2) (layer "F.Cu") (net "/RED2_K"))
 (segment (start 108.2 102.315) (end 101.965 108.55) (width 0.2) (layer "F.Cu") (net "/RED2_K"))
 (segment (start 92.2072 95.2313) (end 92.8213 95.2313) (width 0.2) (layer "F.Cu") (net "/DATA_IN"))
 (segment (start 92.8213 95.2313) (end 93.1 95.51) (width 0.2) (layer "F.Cu") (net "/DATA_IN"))
 (segment (start 99.9517 96.9516) (end 100.5242 96.3791) (width 0.2) (layer "F.Cu") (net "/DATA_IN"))
 (segment (start 97.4117 98.35) (end 97.4117 98.6379) (width 0.2) (layer "F.Cu") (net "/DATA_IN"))
 (segment (start 98.2927 99.5189) (end 99.2623 99.5189) (width 0.2) (layer "F.Cu") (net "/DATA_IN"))
 (segment (start 96.26 98.35) (end 97.4117 98.35) (width 0.2) (layer "F.Cu") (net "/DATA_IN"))
 (segment (start 97.4117 98.6379) (end 98.2927 99.5189) (width 0.2) (layer "F.Cu") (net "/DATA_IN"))
 (segment (start 99.2623 99.5189) (end 99.9517 98.8295) (width 0.2) (layer "F.Cu") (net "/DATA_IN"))
 (segment (start 99.9517 98.8295) (end 99.9517 96.9516) (width 0.2) (layer "F.Cu") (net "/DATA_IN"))
 (via (at 92.2072 95.2313) (size 0.6) (drill 0.3) (layers "F.Cu" "B.Cu") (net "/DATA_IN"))
 (via (at 100.5242 96.3791) (size 0.6) (drill 0.3) (layers "F.Cu" "B.Cu") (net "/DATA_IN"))
 (segment (start 92.2072 95.1079) (end 92.2072 95.2313) (width 0.2) (layer "B.Cu") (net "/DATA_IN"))
 (segment (start 93.9647 93.3504) (end 92.2072 95.1079) (width 0.2) (layer "B.Cu") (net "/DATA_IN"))
 (segment (start 100.5242 96.3791) (end 97.4955 93.3504) (width 0.2) (layer "B.Cu") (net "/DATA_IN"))
 (segment (start 97.4955 93.3504) (end 93.9647 93.3504) (width 0.2) (layer "B.Cu") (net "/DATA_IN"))
 (segment (start 98.035 93) (end 98.035 94.2) (width 0.4) (layer "F.Cu") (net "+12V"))
 (segment (start 94.225 105.9) (end 93.375 105.05) (width 0.4) (layer "F.Cu") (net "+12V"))
 (segment (start 98.035 94.2) (end 98.035 95.4) (width 0.4) (layer "F.Cu") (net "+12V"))
 (segment (start 98.8 98.35) (end 98.8 96.165) (width 0.4) (layer "F.Cu") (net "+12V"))
 (segment (start 98.035 93) (end 98.035 91.8) (width 0.4) (layer "F.Cu") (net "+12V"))
 (segment (start 93.375 105.05) (end 93.375 104.05) (width 0.4) (layer "F.Cu") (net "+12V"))
 (segment (start 98.8 96.165) (end 98.035 95.4) (width 0.4) (layer "F.Cu") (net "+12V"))
 (segment (start 93.375 104.05) (end 93.375 103.0619) (width 0.4) (layer "F.Cu") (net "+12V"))
 (via (at 93.375 103.0619) (size 0.6) (drill 0.3) (layers "F.Cu" "B.Cu") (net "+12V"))
 (segment (start 98.6665 100.7202) (end 98.6665 101.8415) (width 0.4) (layer "B.Cu") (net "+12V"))
 (segment (start 98.8 98.35) (end 98.6665 98.4835) (width 0.4) (layer "B.Cu") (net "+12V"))
 (segment (start 98.6665 101.8415) (end 98.8 101.975) (width 0.4) (layer "B.Cu") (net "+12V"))
 (segment (start 95.7167 100.7202) (end 98.6665 100.7202) (width 0.4) (layer "B.Cu") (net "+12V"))
 (segment (start 98.6665 98.4835) (end 98.6665 100.7202) (width 0.4) (layer "B.Cu") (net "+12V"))
 (segment (start 93.375 103.0619) (end 95.7167 100.7202) (width 0.4) (layer "B.Cu") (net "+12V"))
 (segment (start 95.54 107.6) (end 96.49 108.55) (width 0.2) (layer "F.Cu") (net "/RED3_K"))
 (segment (start 96.49 108.55) (end 98.035 108.55) (width 0.2) (layer "F.Cu") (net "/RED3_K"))
 (segment (start 94.31 97.5) (end 94.7594 97.9494) (width 0.2) (layer "F.Cu") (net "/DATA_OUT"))
 (segment (start 100.4373 99.9206) (end 101.34 100.8233) (width 0.2) (layer "F.Cu") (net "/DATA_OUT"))
 (segment (start 94.7594 99.0288) (end 95.6512 99.9206) (width 0.2) (layer "F.Cu") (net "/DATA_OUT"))
 (segment (start 94.7594 97.9494) (end 94.7594 99.0288) (width 0.2) (layer "F.Cu") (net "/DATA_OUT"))
 (segment (start 95.6512 99.9206) (end 100.4373 99.9206) (width 0.2) (layer "F.Cu") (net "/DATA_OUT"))
 (segment (start 101.34 101.975) (end 101.34 100.8233) (width 0.2) (layer "F.Cu") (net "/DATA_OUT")))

